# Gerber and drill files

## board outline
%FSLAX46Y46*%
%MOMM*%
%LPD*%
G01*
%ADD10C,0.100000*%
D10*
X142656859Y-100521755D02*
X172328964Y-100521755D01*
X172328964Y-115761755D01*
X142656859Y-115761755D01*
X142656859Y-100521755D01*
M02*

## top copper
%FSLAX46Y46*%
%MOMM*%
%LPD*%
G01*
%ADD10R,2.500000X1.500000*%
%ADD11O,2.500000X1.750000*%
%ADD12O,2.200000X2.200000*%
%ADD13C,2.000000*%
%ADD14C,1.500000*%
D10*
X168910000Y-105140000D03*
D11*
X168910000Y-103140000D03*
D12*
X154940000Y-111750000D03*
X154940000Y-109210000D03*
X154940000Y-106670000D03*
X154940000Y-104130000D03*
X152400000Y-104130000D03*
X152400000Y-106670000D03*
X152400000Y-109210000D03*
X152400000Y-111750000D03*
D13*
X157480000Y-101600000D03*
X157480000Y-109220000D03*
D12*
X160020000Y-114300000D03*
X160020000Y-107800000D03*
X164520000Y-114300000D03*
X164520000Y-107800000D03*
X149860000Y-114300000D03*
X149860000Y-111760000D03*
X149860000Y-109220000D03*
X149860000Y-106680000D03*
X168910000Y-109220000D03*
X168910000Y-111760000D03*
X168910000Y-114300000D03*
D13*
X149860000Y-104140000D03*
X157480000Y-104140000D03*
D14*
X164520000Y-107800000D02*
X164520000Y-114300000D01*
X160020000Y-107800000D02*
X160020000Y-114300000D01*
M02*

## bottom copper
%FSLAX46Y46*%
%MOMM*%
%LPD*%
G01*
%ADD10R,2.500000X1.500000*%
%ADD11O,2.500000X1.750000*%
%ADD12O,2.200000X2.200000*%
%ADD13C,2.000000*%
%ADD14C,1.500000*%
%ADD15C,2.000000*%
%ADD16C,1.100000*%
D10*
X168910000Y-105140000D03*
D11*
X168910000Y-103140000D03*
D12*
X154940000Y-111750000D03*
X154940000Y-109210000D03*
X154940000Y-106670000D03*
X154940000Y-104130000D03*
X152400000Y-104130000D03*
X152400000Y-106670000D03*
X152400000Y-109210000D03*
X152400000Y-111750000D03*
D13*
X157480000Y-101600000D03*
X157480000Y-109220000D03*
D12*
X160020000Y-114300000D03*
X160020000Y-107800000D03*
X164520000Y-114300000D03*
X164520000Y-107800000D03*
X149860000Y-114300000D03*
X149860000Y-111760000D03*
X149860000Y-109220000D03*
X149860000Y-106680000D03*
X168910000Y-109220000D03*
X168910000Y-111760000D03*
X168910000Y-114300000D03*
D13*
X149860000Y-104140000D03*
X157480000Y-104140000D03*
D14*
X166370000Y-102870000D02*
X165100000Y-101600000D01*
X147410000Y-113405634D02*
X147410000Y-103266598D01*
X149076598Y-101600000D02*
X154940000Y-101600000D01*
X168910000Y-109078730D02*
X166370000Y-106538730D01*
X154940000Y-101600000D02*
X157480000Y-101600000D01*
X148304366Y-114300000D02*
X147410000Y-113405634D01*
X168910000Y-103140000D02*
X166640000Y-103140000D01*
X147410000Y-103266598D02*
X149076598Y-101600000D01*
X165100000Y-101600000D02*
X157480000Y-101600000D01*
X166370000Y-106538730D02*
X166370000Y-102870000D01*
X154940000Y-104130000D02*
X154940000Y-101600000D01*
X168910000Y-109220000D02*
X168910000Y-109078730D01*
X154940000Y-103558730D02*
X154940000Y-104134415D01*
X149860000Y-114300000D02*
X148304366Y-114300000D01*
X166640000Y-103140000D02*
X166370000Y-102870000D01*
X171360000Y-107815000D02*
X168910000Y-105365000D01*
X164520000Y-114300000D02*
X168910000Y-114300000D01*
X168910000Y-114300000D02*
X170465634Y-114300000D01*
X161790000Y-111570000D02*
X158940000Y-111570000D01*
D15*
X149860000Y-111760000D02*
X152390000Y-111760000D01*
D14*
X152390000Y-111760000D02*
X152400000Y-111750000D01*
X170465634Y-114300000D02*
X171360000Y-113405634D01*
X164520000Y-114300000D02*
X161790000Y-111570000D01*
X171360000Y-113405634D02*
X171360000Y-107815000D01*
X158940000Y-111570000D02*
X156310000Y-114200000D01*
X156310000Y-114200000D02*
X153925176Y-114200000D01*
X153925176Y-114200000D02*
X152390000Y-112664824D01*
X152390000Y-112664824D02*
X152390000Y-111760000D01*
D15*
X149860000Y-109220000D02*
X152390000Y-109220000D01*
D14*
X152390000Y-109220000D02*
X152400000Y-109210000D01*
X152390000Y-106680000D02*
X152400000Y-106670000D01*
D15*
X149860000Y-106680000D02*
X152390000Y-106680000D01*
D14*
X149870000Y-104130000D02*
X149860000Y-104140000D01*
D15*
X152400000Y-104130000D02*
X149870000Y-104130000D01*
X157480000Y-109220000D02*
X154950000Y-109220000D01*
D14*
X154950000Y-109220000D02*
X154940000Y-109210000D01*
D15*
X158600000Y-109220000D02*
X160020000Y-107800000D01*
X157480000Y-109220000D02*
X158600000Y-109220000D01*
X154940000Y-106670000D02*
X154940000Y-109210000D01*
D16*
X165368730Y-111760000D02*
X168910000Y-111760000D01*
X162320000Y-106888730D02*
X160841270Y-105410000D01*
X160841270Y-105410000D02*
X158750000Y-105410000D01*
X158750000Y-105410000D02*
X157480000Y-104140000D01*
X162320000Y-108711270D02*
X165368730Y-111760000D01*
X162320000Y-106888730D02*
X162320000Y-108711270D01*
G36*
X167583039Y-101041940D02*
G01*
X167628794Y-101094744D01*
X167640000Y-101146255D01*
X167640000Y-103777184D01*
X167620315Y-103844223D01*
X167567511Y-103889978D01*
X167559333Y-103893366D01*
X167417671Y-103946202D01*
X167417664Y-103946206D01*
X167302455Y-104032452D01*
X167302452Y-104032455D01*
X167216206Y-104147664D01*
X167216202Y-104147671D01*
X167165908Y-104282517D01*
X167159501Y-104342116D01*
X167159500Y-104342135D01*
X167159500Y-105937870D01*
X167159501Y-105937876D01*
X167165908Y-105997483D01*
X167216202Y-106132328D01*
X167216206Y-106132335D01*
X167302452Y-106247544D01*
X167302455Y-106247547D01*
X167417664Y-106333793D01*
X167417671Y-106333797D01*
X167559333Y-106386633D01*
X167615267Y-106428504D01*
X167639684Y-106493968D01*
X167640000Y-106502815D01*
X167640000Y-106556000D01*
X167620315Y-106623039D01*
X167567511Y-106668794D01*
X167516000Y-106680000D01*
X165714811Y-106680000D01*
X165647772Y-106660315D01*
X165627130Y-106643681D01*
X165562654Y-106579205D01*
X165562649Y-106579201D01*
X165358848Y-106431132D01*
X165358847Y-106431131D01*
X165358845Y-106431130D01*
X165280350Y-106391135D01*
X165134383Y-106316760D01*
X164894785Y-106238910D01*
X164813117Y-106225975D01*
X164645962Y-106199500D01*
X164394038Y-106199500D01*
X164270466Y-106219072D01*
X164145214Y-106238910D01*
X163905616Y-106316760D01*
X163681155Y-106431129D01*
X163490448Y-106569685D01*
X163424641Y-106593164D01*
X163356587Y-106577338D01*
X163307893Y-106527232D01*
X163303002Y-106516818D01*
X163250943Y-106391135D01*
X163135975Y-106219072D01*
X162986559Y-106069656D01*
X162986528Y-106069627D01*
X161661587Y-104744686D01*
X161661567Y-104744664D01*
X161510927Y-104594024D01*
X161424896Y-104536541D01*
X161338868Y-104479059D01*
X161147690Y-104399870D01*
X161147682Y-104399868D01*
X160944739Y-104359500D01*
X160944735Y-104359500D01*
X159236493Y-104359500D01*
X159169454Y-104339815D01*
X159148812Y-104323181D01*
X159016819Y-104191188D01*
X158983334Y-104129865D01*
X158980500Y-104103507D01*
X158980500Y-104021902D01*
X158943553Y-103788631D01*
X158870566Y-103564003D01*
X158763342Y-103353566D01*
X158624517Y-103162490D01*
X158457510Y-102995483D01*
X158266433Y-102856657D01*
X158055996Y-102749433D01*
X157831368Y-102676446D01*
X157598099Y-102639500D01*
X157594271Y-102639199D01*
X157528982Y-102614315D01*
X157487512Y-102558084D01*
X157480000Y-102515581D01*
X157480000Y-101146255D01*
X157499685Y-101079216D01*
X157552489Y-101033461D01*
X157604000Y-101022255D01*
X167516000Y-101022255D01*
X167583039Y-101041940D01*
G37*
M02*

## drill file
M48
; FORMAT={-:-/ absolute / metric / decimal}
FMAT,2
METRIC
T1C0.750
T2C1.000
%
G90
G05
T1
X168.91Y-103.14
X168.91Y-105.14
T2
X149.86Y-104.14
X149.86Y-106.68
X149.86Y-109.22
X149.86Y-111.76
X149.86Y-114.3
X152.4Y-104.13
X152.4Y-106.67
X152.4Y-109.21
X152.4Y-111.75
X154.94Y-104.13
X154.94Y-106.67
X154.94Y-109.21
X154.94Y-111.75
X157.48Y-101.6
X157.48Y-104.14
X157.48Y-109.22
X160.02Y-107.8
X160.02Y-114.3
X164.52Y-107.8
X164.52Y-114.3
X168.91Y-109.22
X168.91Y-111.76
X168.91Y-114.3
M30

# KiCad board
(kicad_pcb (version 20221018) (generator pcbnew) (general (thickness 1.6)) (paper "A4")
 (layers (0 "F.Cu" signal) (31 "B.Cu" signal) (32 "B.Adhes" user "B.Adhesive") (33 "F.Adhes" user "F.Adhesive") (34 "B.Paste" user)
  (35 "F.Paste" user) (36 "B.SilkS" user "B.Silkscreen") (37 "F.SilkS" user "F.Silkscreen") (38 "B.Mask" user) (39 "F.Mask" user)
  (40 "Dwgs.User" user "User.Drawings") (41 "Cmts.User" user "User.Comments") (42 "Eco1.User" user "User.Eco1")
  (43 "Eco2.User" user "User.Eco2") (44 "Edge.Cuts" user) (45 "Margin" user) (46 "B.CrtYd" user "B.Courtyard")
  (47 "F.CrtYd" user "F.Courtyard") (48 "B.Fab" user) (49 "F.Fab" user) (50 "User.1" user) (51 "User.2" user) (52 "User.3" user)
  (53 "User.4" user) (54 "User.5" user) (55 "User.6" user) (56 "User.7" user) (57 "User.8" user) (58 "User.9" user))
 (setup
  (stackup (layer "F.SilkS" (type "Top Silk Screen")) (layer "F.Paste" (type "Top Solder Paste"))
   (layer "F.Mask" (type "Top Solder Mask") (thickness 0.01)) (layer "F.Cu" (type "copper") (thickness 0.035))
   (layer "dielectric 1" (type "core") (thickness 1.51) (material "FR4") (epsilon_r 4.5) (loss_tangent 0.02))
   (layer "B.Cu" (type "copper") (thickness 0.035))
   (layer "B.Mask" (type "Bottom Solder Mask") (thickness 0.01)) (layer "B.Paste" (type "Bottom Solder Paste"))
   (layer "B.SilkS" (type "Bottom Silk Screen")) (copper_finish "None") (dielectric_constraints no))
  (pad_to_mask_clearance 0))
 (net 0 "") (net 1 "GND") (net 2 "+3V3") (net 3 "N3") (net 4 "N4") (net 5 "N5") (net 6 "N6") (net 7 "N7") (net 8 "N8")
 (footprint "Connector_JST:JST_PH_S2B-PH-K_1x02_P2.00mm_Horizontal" (layer "F.Cu") (at 168.91 105.14 90)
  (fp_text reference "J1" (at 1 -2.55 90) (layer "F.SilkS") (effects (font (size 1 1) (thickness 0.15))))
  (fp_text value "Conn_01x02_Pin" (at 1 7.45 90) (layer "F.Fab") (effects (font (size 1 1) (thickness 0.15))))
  (pad "1" thru_hole rect (at 0 0 90) (size 1.5 2.5) (drill 0.75) (layers "*.Cu" "*.Mask") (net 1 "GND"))
  (pad "2" thru_hole oval (at 2 0 90) (size 1.75 2.5) (drill 0.75) (layers "*.Cu" "*.Mask") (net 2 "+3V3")))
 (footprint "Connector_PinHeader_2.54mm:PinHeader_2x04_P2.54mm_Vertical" (layer "F.Cu") (at 154.94 111.75 180)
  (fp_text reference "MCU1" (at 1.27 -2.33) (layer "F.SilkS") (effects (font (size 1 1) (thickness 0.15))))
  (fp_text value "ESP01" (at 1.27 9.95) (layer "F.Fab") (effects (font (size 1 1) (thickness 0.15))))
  (pad "1" thru_hole oval (at 0 0 180) (size 2.2 2.2) (drill 1) (layers "*.Cu" "*.Mask") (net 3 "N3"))
  (pad "2" thru_hole oval (at 0 2.54 180) (size 2.2 2.2) (drill 1) (layers "*.Cu" "*.Mask") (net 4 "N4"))
  (pad "3" thru_hole oval (at 0 5.08 180) (size 2.2 2.2) (drill 1) (layers "*.Cu" "*.Mask") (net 4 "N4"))
  (pad "4" thru_hole oval (at 0 7.62 180) (size 2.2 2.2) (drill 1) (layers "*.Cu" "*.Mask") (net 2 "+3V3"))
  (pad "5" thru_hole oval (at 2.54 7.62 180) (size 2.2 2.2) (drill 1) (layers "*.Cu" "*.Mask") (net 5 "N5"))
  (pad "6" thru_hole oval (at 2.54 5.08 180) (size 2.2 2.2) (drill 1) (layers "*.Cu" "*.Mask") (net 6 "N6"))
  (pad "7" thru_hole oval (at 2.54 2.54 180) (size 2.2 2.2) (drill 1) (layers "*.Cu" "*.Mask") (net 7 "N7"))
  (pad "8" thru_hole oval (at 2.54 0 180) (size 2.2 2.2) (drill 1) (layers "*.Cu" "*.Mask") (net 1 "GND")))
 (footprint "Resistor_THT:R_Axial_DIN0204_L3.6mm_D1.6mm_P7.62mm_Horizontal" (layer "F.Cu") (at 157.48 101.6 -90)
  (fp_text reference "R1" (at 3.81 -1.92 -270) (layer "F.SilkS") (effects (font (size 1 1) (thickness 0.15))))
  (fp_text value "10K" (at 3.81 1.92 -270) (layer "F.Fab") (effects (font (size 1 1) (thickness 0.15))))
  (pad "1" thru_hole circle (at 0 0 270) (size 2 2) (drill 1) (layers "*.Cu" "*.Mask") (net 2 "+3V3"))
  (pad "2" thru_hole circle (at 7.62 0 270) (size 2 2) (drill 1) (layers "*.Cu" "*.Mask") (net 4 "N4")))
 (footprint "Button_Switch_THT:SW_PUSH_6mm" (layer "F.Cu") (at 160.02 114.3 90)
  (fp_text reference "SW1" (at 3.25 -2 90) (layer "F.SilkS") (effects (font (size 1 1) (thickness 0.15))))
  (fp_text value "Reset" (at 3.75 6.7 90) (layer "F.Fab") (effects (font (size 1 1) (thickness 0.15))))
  (pad "1" thru_hole oval (at 0 0 90) (size 2.2 2.2) (drill 1) (layers "*.Cu" "*.Mask") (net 4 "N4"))
  (pad "1" thru_hole oval (at 6.5 0 90) (size 2.2 2.2) (drill 1) (layers "*.Cu" "*.Mask") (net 4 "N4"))
  (pad "2" thru_hole oval (at 0 4.5 90) (size 2.2 2.2) (drill 1) (layers "*.Cu" "*.Mask") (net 1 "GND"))
  (pad "2" thru_hole oval (at 6.5 4.5 90) (size 2.2 2.2) (drill 1) (layers "*.Cu" "*.Mask") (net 1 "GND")))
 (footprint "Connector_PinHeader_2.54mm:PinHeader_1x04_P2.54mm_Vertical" (layer "F.Cu") (at 149.86 114.3 180)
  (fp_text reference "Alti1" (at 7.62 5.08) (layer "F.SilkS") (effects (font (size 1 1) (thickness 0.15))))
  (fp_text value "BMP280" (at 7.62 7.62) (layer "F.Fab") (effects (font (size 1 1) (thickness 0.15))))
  (pad "1" thru_hole oval (at 0 0 180) (size 2.2 2.2) (drill 1) (layers "*.Cu" "*.Mask") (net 2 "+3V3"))
  (pad "2" thru_hole oval (at 0 2.54 180) (size 2.2 2.2) (drill 1) (layers "*.Cu" "*.Mask") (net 1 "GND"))
  (pad "3" thru_hole oval (at 0 5.08 180) (size 2.2 2.2) (drill 1) (layers "*.Cu" "*.Mask") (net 7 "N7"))
  (pad "4" thru_hole oval (at 0 7.62 180) (size 2.2 2.2) (drill 1) (layers "*.Cu" "*.Mask") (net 6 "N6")))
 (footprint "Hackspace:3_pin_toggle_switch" (layer "B.Cu") (at 168.91 111.76 180)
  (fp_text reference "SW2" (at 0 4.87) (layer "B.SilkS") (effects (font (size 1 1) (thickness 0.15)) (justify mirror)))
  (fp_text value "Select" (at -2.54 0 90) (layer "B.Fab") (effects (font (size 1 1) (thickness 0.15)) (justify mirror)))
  (pad "1" thru_hole oval (at 0 2.54 180) (size 2.2 2.2) (drill 1) (layers "*.Cu" "*.Mask") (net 2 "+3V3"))
  (pad "2" thru_hole oval (at 0 0 180) (size 2.2 2.2) (drill 1) (layers "*.Cu" "*.Mask") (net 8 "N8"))
  (pad "3" thru_hole oval (at 0 -2.54 180) (size 2.2 2.2) (drill 1) (layers "*.Cu" "*.Mask") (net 1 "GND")))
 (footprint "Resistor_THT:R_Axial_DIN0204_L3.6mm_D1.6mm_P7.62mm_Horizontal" (layer "B.Cu") (at 149.86 104.14)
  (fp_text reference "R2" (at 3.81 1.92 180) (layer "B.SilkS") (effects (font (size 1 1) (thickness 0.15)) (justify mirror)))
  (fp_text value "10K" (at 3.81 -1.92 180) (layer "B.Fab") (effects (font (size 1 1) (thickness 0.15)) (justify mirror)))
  (pad "1" thru_hole circle (at 0 0) (size 2 2) (drill 1) (layers "*.Cu" "*.Mask") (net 5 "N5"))
  (pad "2" thru_hole circle (at 7.62 0) (size 2 2) (drill 1) (layers "*.Cu" "*.Mask") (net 8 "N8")))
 (gr_rect (start 142.656859 100.521755) (end 172.328964 115.761755) (stroke (width 0.1) (type default)) (fill none) (layer "Edge.Cuts"))
 (segment (start 166.37 102.87) (end 165.1 101.6) (width 1.5) (layer "B.Cu") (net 2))
 (segment (start 147.41 113.405634) (end 147.41 103.266598) (width 1.5) (layer "B.Cu") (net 2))
 (segment (start 149.076598 101.6) (end 154.94 101.6) (width 1.5) (layer "B.Cu") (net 2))
 (segment (start 168.91 109.07873) (end 166.37 106.53873) (width 1.5) (layer "B.Cu") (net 2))
 (segment (start 154.94 101.6) (end 157.48 101.6) (width 1.5) (layer "B.Cu") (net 2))
 (segment (start 148.304366 114.3) (end 147.41 113.405634) (width 1.5) (layer "B.Cu") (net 2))
 (segment (start 168.91 103.14) (end 166.64 103.14) (width 1.5) (layer "B.Cu") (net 2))
 (segment (start 147.41 103.266598) (end 149.076598 101.6) (width 1.5) (layer "B.Cu") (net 2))
 (segment (start 165.1 101.6) (end 157.48 101.6) (width 1.5) (layer "B.Cu") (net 2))
 (segment (start 166.37 106.53873) (end 166.37 102.87) (width 1.5) (layer "B.Cu") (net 2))
 (segment (start 154.94 104.13) (end 154.94 101.6) (width 1.5) (layer "B.Cu") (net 2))
 (segment (start 168.91 109.22) (end 168.91 109.07873) (width 1.5) (layer "B.Cu") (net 2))
 (segment (start 154.94 103.55873) (end 154.94 104.134415) (width 1.5) (layer "B.Cu") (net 2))
 (segment (start 149.86 114.3) (end 148.304366 114.3) (width 1.5) (layer "B.Cu") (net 2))
 (segment (start 166.64 103.14) (end 166.37 102.87) (width 1.5) (layer "B.Cu") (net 2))
 (segment (start 164.52 107.8) (end 164.52 114.3) (width 1.5) (layer "F.Cu") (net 1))
 (segment (start 171.36 107.815) (end 168.91 105.365) (width 1.5) (layer "B.Cu") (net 1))
 (segment (start 164.52 114.3) (end 168.91 114.3) (width 1.5) (layer "B.Cu") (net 1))
 (segment (start 168.91 114.3) (end 170.465634 114.3) (width 1.5) (layer "B.Cu") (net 1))
 (segment (start 161.79 111.57) (end 158.94 111.57) (width 1.5) (layer "B.Cu") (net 1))
 (segment (start 149.86 111.76) (end 152.39 111.76) (width 2) (layer "B.Cu") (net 1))
 (segment (start 152.39 111.76) (end 152.4 111.75) (width 1.5) (layer "B.Cu") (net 1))
 (segment (start 170.465634 114.3) (end 171.36 113.405634) (width 1.5) (layer "B.Cu") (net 1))
 (segment (start 164.52 114.3) (end 161.79 111.57) (width 1.5) (layer "B.Cu") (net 1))
 (segment (start 171.36 113.405634) (end 171.36 107.815) (width 1.5) (layer "B.Cu") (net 1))
 (segment (start 158.94 111.57) (end 156.31 114.2) (width 1.5) (layer "B.Cu") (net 1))
 (segment (start 156.31 114.2) (end 153.925176 114.2) (width 1.5) (layer "B.Cu") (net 1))
 (segment (start 153.925176 114.2) (end 152.39 112.664824) (width 1.5) (layer "B.Cu") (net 1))
 (segment (start 152.39 112.664824) (end 152.39 111.76) (width 1.5) (layer "B.Cu") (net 1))
 (segment (start 149.86 109.22) (end 152.39 109.22) (width 2) (layer "B.Cu") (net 7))
 (segment (start 152.39 109.22) (end 152.4 109.21) (width 1.5) (layer "B.Cu") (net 7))
 (segment (start 152.39 106.68) (end 152.4 106.67) (width 1.5) (layer "B.Cu") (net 6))
 (segment (start 149.86 106.68) (end 152.39 106.68) (width 2) (layer "B.Cu") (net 6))
 (segment (start 149.87 104.13) (end 149.86 104.14) (width 1.5) (layer "B.Cu") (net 5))
 (segment (start 152.4 104.13) (end 149.87 104.13) (width 2) (layer "B.Cu") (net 5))
 (segment (start 160.02 107.8) (end 160.02 114.3) (width 1.5) (layer "F.Cu") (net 4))
 (segment (start 157.48 109.22) (end 154.95 109.22) (width 2) (layer "B.Cu") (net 4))
 (segment (start 154.95 109.22) (end 154.94 109.21) (width 1.5) (layer "B.Cu") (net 4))
 (segment (start 158.6 109.22) (end 160.02 107.8) (width 2) (layer "B.Cu") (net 4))
 (segment (start 157.48 109.22) (end 158.6 109.22) (width 2) (layer "B.Cu") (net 4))
 (segment (start 154.94 106.67) (end 154.94 109.21) (width 2) (layer "B.Cu") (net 4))
 (segment (start 165.36873 111.76) (end 168.91 111.76) (width 1.1) (layer "B.Cu") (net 8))
 (segment (start 162.32 106.88873) (end 160.84127 105.41) (width 1.1) (layer "B.Cu") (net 8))
 (segment (start 160.84127 105.41) (end 158.75 105.41) (width 1.1) (layer "B.Cu") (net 8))
 (segment (start 158.75 105.41) (end 157.48 104.14) (width 1.1) (layer "B.Cu") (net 8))
 (segment (start 162.32 108.71127) (end 165.36873 111.76) (width 1.1) (layer "B.Cu") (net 8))
 (segment (start 162.32 106.88873) (end 162.32 108.71127) (width 1.1) (layer "B.Cu") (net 8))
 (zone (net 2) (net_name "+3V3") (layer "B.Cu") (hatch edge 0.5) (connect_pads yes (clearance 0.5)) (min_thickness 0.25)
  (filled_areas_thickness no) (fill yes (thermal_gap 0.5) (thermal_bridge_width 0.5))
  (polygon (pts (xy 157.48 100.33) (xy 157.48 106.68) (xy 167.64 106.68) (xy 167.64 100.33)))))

